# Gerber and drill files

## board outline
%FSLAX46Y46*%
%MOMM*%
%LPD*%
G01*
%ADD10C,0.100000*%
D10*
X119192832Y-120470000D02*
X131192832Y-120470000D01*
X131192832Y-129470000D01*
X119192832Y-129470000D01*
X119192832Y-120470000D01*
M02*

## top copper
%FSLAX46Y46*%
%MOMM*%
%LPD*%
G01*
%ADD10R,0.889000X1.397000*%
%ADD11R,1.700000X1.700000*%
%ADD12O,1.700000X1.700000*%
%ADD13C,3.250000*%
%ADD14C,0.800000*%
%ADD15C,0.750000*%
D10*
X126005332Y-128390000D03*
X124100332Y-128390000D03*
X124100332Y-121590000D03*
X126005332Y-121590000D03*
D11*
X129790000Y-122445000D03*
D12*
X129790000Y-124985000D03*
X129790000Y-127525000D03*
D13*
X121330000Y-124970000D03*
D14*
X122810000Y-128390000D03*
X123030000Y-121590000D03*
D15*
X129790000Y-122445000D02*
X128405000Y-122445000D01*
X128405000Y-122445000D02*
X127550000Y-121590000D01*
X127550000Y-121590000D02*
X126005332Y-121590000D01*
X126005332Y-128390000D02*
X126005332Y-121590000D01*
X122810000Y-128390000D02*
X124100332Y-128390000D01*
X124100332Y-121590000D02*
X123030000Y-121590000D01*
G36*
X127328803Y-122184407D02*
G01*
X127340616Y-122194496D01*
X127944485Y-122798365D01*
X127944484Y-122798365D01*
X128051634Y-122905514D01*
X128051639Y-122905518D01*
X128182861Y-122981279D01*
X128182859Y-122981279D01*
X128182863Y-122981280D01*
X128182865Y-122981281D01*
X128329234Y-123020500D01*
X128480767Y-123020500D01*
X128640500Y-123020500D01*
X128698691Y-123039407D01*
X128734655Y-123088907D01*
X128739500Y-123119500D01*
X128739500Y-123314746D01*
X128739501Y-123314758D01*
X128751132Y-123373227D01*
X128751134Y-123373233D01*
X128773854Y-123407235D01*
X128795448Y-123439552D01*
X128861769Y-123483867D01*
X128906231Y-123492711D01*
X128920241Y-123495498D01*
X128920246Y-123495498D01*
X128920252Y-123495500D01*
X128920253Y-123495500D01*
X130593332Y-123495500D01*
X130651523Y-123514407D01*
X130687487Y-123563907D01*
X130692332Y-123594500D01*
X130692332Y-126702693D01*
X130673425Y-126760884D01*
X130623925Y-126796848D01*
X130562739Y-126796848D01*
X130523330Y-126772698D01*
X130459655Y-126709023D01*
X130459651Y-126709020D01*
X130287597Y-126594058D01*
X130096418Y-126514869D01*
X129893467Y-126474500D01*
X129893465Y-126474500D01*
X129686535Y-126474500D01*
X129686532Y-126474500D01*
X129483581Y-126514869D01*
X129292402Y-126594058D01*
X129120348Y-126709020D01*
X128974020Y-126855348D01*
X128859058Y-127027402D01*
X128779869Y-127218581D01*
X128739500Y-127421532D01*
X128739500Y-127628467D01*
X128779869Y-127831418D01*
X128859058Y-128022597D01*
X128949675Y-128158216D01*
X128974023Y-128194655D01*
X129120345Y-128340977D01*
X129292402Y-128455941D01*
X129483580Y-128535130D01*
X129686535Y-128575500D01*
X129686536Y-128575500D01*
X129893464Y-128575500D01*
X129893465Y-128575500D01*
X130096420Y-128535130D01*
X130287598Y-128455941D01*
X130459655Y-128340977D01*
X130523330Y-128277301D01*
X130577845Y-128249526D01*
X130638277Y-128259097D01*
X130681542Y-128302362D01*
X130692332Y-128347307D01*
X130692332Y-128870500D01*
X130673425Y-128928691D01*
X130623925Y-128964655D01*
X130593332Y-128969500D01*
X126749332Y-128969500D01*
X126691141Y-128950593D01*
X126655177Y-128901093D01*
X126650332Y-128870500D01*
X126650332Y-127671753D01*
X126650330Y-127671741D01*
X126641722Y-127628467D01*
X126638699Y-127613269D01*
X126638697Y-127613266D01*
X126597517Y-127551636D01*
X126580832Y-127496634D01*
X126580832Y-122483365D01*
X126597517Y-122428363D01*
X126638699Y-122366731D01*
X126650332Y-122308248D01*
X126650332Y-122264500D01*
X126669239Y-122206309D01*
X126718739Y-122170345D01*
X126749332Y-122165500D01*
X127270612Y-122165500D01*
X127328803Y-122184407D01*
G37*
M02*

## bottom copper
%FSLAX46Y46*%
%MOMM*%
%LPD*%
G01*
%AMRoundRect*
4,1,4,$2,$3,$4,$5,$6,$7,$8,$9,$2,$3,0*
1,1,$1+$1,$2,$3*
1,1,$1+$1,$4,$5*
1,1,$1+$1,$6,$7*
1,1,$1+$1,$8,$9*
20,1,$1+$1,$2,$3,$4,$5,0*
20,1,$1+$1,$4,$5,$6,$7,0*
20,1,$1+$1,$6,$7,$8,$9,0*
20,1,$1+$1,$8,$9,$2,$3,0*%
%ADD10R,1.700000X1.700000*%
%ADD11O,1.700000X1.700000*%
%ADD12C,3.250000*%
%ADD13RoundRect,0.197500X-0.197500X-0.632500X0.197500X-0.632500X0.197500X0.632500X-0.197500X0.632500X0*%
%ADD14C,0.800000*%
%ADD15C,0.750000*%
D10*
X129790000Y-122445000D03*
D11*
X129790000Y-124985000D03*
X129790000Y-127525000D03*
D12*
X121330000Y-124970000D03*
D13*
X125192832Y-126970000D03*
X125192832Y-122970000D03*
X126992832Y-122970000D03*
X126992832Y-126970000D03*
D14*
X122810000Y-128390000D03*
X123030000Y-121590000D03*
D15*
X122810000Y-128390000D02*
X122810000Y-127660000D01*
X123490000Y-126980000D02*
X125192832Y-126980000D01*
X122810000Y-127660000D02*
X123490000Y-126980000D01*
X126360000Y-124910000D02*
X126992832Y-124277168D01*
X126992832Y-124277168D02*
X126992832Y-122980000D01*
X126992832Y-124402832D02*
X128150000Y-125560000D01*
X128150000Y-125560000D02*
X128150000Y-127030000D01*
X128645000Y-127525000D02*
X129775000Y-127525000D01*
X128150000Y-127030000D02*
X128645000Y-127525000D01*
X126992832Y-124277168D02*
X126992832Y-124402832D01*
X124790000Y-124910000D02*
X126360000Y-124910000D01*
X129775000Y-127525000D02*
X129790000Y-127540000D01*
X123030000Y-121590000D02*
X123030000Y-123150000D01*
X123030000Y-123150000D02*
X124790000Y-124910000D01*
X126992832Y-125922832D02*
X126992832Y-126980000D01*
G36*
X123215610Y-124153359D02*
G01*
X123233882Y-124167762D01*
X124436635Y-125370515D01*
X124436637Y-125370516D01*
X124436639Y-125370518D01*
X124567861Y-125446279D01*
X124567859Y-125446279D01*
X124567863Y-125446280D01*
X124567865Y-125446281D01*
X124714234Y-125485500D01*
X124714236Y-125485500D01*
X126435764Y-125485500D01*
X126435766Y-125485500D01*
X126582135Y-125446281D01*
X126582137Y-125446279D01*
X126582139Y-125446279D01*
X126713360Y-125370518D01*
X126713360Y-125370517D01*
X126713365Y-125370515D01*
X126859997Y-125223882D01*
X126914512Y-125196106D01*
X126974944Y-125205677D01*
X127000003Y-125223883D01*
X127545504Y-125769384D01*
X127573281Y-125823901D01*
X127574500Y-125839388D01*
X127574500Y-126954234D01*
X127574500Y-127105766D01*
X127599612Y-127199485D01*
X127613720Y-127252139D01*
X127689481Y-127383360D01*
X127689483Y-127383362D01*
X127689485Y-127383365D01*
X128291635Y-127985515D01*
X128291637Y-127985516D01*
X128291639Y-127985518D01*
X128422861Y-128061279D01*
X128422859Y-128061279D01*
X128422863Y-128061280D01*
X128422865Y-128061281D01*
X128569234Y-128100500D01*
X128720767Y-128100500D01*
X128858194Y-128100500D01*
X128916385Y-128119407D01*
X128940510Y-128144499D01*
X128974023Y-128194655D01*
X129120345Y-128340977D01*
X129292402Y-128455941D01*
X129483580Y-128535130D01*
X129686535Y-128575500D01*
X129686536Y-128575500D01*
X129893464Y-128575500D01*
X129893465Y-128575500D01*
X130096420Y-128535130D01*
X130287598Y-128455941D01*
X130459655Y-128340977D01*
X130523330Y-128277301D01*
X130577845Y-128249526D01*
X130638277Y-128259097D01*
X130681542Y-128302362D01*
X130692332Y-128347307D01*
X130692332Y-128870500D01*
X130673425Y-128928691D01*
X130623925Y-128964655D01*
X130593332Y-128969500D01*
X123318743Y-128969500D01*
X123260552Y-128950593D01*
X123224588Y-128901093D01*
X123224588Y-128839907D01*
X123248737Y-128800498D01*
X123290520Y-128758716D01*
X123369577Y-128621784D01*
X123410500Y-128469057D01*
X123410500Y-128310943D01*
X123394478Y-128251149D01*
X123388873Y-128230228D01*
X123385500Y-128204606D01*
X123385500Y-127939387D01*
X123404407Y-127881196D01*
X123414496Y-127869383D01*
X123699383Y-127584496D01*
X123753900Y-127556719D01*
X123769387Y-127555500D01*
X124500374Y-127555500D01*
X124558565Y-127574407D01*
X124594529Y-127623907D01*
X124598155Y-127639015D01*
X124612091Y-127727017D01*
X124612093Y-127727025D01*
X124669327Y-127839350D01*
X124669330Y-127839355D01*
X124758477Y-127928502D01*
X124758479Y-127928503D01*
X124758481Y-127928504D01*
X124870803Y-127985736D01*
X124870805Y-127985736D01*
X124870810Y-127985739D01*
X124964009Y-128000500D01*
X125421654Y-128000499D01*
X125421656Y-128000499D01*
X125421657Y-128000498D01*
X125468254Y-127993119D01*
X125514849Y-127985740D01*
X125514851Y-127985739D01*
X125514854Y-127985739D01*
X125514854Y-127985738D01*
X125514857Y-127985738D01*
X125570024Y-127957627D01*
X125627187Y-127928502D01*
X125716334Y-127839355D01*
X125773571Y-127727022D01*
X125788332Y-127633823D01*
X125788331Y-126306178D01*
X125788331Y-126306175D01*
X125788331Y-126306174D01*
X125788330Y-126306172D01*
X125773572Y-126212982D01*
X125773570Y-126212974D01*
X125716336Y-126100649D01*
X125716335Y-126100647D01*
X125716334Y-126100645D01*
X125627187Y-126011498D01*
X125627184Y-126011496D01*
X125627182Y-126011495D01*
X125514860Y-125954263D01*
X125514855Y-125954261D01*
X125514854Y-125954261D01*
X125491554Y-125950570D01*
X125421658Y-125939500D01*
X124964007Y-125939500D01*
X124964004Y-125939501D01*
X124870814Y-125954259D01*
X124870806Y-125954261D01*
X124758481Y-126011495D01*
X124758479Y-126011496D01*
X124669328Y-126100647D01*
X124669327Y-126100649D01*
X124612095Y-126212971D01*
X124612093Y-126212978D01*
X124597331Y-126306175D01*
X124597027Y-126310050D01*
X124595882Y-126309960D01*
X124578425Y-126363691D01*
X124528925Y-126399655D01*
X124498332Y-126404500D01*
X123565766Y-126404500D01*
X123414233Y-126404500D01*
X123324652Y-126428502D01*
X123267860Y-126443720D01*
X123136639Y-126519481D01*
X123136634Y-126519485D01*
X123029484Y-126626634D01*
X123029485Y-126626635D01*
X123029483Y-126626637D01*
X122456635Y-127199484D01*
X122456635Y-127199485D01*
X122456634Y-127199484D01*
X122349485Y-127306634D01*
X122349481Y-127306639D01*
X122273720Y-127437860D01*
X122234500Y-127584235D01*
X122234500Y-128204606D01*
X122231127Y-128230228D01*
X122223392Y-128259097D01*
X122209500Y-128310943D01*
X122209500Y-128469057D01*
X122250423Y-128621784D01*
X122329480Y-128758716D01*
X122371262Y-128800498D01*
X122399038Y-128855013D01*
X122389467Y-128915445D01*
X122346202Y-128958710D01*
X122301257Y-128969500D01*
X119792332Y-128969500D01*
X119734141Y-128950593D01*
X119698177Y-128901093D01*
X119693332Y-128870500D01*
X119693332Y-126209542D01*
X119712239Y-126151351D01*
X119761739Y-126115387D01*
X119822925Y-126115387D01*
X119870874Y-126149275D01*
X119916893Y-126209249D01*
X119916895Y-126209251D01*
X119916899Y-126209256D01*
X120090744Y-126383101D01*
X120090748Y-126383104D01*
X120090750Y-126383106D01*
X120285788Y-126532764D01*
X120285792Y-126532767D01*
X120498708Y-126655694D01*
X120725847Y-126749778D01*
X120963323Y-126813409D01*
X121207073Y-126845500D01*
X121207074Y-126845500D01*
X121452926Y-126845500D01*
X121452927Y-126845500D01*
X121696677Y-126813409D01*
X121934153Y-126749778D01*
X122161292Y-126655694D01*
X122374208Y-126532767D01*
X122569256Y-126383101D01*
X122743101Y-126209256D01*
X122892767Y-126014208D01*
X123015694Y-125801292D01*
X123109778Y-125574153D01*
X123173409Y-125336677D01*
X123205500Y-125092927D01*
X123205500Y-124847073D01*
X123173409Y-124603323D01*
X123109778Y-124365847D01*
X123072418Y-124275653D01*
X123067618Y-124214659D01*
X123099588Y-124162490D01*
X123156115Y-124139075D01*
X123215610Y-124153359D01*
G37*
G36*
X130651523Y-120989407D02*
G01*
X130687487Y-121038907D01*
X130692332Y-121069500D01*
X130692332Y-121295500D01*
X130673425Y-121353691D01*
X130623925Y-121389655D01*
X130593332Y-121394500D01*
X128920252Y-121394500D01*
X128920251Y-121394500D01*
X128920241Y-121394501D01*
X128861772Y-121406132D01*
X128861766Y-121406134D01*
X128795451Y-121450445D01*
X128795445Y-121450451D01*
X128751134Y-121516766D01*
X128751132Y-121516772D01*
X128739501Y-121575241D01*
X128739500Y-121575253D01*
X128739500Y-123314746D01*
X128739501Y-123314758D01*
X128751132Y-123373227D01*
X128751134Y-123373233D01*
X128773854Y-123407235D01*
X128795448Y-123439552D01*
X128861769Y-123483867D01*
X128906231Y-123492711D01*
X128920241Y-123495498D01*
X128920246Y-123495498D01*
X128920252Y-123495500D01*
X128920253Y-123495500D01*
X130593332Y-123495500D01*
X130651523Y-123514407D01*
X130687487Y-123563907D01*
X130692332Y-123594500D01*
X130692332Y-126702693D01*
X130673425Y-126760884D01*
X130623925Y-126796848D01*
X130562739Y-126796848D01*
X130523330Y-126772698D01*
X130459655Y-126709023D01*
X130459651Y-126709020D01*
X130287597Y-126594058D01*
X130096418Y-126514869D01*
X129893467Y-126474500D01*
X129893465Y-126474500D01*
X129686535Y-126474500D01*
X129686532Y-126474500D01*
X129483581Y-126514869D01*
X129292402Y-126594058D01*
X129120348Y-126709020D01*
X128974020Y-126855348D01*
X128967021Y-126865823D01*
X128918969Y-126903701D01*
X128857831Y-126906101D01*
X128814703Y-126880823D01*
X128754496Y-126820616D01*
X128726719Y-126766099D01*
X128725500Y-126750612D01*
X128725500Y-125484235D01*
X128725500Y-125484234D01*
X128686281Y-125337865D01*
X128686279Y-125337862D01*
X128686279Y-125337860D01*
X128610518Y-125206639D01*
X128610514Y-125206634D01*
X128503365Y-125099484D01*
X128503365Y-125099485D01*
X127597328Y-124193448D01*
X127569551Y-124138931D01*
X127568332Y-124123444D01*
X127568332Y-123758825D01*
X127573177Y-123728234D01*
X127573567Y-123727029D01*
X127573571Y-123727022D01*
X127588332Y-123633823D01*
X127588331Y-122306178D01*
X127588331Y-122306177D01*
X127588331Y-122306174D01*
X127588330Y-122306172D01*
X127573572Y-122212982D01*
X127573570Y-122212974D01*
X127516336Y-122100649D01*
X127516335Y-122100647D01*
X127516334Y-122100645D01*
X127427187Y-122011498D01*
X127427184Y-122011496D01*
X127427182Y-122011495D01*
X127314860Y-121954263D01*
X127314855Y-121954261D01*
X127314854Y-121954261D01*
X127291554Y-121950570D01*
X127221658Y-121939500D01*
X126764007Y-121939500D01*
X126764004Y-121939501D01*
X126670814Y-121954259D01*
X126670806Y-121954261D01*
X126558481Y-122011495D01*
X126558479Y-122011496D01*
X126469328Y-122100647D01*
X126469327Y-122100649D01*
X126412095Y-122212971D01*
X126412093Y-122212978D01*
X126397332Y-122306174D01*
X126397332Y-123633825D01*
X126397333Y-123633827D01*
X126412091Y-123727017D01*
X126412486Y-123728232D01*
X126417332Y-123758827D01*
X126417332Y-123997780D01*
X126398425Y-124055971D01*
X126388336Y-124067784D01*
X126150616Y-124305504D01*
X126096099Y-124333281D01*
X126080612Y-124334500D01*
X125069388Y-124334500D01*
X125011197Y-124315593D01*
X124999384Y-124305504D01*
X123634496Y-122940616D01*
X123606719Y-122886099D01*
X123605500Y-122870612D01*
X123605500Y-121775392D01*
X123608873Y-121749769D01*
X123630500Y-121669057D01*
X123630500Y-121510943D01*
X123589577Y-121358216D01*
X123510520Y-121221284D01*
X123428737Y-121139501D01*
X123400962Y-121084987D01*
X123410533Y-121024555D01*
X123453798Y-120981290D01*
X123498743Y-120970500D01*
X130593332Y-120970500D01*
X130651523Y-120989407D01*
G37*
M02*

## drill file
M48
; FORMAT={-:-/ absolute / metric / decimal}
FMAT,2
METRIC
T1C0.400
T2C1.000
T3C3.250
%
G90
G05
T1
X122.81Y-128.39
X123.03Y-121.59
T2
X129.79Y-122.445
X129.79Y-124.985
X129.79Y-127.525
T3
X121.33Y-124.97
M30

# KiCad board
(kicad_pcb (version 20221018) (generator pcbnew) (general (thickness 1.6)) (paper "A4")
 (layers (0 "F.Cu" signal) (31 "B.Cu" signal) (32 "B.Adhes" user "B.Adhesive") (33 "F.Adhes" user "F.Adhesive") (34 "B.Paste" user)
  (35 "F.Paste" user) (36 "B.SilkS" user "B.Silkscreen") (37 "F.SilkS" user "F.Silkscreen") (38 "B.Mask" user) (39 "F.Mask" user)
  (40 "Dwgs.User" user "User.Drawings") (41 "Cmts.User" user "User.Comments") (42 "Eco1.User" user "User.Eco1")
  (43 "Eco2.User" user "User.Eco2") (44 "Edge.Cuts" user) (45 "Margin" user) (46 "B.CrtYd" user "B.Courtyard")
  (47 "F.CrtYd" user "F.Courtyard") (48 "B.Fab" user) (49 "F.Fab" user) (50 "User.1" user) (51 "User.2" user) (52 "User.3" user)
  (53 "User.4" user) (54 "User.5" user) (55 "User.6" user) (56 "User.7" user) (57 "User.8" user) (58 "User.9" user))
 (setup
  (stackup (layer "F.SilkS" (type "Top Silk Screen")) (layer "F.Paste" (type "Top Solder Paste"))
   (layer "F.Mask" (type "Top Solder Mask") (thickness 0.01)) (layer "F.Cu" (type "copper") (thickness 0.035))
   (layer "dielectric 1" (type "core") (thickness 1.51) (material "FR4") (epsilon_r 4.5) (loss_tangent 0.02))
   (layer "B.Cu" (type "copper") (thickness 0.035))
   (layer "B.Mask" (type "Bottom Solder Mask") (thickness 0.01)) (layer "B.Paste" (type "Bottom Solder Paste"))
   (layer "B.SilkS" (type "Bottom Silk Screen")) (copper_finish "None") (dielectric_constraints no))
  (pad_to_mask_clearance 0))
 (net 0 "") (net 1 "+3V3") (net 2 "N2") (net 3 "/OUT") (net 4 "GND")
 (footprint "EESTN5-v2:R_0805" (layer "F.Cu") (at 125.052832 128.39 180)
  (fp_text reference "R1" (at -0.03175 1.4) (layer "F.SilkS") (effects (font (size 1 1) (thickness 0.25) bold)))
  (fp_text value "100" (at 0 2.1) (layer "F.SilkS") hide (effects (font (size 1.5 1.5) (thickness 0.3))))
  (pad "1" smd rect (at -0.9525 0 180) (size 0.889 1.397) (layers "F.Cu" "F.Paste" "F.Mask") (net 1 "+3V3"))
  (pad "2" smd rect (at 0.9525 0 180) (size 0.889 1.397) (layers "F.Cu" "F.Paste" "F.Mask") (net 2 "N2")))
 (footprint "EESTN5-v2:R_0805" (layer "F.Cu") (at 125.052832 121.59)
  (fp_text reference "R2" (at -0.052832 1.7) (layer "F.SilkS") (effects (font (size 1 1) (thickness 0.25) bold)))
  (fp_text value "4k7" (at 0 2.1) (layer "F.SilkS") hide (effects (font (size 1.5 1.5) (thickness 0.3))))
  (pad "1" smd rect (at -0.9525 0) (size 0.889 1.397) (layers "F.Cu" "F.Paste" "F.Mask") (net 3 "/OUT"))
  (pad "2" smd rect (at 0.9525 0) (size 0.889 1.397) (layers "F.Cu" "F.Paste" "F.Mask") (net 1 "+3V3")))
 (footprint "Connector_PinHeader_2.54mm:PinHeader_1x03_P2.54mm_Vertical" (layer "F.Cu") (at 129.79 122.445)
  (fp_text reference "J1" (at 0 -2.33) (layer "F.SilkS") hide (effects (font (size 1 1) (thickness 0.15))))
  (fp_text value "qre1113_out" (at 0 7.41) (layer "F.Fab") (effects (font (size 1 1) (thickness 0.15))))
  (pad "1" thru_hole rect (at 0 0) (size 1.7 1.7) (drill 1) (layers "*.Cu" "*.Mask") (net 1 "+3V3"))
  (pad "2" thru_hole oval (at 0 2.54) (size 1.7 1.7) (drill 1) (layers "*.Cu" "*.Mask") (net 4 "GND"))
  (pad "3" thru_hole oval (at 0 5.08) (size 1.7 1.7) (drill 1) (layers "*.Cu" "*.Mask") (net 3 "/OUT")))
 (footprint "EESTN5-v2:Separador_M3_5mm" (layer "F.Cu") (at 121.33 124.97 180)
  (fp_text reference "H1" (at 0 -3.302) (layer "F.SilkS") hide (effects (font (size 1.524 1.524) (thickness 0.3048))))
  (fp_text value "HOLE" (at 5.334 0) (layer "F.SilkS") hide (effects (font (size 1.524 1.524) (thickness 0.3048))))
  (pad "1" thru_hole circle (at 0 0 180) (size 3.25 3.25) (drill 3.25) (layers "*.Cu" "F.SilkS")))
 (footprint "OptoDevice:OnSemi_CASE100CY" (layer "B.Cu") (at 126.092832 124.97)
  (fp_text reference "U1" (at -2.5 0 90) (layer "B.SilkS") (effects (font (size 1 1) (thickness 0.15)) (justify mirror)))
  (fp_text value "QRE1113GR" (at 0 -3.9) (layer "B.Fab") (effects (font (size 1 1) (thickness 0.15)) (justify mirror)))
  (pad "1" smd roundrect (at -0.9 2) (size 0.79 1.66) (layers "B.Cu" "B.Paste" "B.Mask") (roundrect_rratio 0.25) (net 2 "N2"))
  (pad "2" smd roundrect (at -0.9 -2) (size 0.79 1.66) (layers "B.Cu" "B.Paste" "B.Mask") (roundrect_rratio 0.25) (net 4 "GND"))
  (pad "3" smd roundrect (at 0.9 -2) (size 0.79 1.66) (layers "B.Cu" "B.Paste" "B.Mask") (roundrect_rratio 0.25) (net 3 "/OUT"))
  (pad "4" smd roundrect (at 0.9 2) (size 0.79 1.66) (layers "B.Cu" "B.Paste" "B.Mask") (roundrect_rratio 0.25) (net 4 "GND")))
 (gr_rect (start 131.192832 120.47) (end 119.192832 129.47) (stroke (width 0.1) (type default)) (fill none) (layer "Edge.Cuts"))
 (segment (start 129.79 122.445) (end 128.405 122.445) (width 0.75) (layer "F.Cu") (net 1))
 (segment (start 128.405 122.445) (end 127.55 121.59) (width 0.75) (layer "F.Cu") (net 1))
 (segment (start 127.55 121.59) (end 126.005332 121.59) (width 0.75) (layer "F.Cu") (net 1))
 (segment (start 126.005332 128.39) (end 126.005332 121.59) (width 0.75) (layer "F.Cu") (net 1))
 (segment (start 122.81 128.39) (end 124.100332 128.39) (width 0.75) (layer "F.Cu") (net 2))
 (via (at 122.81 128.39) (size 0.8) (drill 0.4) (layers "F.Cu" "B.Cu") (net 2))
 (segment (start 122.81 128.39) (end 122.81 127.66) (width 0.75) (layer "B.Cu") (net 2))
 (segment (start 123.49 126.98) (end 125.192832 126.98) (width 0.75) (layer "B.Cu") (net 2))
 (segment (start 122.81 127.66) (end 123.49 126.98) (width 0.75) (layer "B.Cu") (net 2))
 (segment (start 124.100332 121.59) (end 123.03 121.59) (width 0.75) (layer "F.Cu") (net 3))
 (via (at 123.03 121.59) (size 0.8) (drill 0.4) (layers "F.Cu" "B.Cu") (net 3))
 (segment (start 126.36 124.91) (end 126.992832 124.277168) (width 0.75) (layer "B.Cu") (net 3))
 (segment (start 126.992832 124.277168) (end 126.992832 122.98) (width 0.75) (layer "B.Cu") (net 3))
 (segment (start 126.992832 124.402832) (end 128.15 125.56) (width 0.75) (layer "B.Cu") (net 3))
 (segment (start 128.15 125.56) (end 128.15 127.03) (width 0.75) (layer "B.Cu") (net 3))
 (segment (start 128.645 127.525) (end 129.775 127.525) (width 0.75) (layer "B.Cu") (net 3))
 (segment (start 128.15 127.03) (end 128.645 127.525) (width 0.75) (layer "B.Cu") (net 3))
 (segment (start 126.992832 124.277168) (end 126.992832 124.402832) (width 0.75) (layer "B.Cu") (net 3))
 (segment (start 124.79 124.91) (end 126.36 124.91) (width 0.75) (layer "B.Cu") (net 3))
 (segment (start 129.775 127.525) (end 129.79 127.54) (width 0.75) (layer "B.Cu") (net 3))
 (segment (start 123.03 121.59) (end 123.03 123.15) (width 0.75) (layer "B.Cu") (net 3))
 (segment (start 123.03 123.15) (end 124.79 124.91) (width 0.75) (layer "B.Cu") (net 3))
 (segment (start 126.992832 125.922832) (end 126.992832 126.98) (width 0.75) (layer "B.Cu") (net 4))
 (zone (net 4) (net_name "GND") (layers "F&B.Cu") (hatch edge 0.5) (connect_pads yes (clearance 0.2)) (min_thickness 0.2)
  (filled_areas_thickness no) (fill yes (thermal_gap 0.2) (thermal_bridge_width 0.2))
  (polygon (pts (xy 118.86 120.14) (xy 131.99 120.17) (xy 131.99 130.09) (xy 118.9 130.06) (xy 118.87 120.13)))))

